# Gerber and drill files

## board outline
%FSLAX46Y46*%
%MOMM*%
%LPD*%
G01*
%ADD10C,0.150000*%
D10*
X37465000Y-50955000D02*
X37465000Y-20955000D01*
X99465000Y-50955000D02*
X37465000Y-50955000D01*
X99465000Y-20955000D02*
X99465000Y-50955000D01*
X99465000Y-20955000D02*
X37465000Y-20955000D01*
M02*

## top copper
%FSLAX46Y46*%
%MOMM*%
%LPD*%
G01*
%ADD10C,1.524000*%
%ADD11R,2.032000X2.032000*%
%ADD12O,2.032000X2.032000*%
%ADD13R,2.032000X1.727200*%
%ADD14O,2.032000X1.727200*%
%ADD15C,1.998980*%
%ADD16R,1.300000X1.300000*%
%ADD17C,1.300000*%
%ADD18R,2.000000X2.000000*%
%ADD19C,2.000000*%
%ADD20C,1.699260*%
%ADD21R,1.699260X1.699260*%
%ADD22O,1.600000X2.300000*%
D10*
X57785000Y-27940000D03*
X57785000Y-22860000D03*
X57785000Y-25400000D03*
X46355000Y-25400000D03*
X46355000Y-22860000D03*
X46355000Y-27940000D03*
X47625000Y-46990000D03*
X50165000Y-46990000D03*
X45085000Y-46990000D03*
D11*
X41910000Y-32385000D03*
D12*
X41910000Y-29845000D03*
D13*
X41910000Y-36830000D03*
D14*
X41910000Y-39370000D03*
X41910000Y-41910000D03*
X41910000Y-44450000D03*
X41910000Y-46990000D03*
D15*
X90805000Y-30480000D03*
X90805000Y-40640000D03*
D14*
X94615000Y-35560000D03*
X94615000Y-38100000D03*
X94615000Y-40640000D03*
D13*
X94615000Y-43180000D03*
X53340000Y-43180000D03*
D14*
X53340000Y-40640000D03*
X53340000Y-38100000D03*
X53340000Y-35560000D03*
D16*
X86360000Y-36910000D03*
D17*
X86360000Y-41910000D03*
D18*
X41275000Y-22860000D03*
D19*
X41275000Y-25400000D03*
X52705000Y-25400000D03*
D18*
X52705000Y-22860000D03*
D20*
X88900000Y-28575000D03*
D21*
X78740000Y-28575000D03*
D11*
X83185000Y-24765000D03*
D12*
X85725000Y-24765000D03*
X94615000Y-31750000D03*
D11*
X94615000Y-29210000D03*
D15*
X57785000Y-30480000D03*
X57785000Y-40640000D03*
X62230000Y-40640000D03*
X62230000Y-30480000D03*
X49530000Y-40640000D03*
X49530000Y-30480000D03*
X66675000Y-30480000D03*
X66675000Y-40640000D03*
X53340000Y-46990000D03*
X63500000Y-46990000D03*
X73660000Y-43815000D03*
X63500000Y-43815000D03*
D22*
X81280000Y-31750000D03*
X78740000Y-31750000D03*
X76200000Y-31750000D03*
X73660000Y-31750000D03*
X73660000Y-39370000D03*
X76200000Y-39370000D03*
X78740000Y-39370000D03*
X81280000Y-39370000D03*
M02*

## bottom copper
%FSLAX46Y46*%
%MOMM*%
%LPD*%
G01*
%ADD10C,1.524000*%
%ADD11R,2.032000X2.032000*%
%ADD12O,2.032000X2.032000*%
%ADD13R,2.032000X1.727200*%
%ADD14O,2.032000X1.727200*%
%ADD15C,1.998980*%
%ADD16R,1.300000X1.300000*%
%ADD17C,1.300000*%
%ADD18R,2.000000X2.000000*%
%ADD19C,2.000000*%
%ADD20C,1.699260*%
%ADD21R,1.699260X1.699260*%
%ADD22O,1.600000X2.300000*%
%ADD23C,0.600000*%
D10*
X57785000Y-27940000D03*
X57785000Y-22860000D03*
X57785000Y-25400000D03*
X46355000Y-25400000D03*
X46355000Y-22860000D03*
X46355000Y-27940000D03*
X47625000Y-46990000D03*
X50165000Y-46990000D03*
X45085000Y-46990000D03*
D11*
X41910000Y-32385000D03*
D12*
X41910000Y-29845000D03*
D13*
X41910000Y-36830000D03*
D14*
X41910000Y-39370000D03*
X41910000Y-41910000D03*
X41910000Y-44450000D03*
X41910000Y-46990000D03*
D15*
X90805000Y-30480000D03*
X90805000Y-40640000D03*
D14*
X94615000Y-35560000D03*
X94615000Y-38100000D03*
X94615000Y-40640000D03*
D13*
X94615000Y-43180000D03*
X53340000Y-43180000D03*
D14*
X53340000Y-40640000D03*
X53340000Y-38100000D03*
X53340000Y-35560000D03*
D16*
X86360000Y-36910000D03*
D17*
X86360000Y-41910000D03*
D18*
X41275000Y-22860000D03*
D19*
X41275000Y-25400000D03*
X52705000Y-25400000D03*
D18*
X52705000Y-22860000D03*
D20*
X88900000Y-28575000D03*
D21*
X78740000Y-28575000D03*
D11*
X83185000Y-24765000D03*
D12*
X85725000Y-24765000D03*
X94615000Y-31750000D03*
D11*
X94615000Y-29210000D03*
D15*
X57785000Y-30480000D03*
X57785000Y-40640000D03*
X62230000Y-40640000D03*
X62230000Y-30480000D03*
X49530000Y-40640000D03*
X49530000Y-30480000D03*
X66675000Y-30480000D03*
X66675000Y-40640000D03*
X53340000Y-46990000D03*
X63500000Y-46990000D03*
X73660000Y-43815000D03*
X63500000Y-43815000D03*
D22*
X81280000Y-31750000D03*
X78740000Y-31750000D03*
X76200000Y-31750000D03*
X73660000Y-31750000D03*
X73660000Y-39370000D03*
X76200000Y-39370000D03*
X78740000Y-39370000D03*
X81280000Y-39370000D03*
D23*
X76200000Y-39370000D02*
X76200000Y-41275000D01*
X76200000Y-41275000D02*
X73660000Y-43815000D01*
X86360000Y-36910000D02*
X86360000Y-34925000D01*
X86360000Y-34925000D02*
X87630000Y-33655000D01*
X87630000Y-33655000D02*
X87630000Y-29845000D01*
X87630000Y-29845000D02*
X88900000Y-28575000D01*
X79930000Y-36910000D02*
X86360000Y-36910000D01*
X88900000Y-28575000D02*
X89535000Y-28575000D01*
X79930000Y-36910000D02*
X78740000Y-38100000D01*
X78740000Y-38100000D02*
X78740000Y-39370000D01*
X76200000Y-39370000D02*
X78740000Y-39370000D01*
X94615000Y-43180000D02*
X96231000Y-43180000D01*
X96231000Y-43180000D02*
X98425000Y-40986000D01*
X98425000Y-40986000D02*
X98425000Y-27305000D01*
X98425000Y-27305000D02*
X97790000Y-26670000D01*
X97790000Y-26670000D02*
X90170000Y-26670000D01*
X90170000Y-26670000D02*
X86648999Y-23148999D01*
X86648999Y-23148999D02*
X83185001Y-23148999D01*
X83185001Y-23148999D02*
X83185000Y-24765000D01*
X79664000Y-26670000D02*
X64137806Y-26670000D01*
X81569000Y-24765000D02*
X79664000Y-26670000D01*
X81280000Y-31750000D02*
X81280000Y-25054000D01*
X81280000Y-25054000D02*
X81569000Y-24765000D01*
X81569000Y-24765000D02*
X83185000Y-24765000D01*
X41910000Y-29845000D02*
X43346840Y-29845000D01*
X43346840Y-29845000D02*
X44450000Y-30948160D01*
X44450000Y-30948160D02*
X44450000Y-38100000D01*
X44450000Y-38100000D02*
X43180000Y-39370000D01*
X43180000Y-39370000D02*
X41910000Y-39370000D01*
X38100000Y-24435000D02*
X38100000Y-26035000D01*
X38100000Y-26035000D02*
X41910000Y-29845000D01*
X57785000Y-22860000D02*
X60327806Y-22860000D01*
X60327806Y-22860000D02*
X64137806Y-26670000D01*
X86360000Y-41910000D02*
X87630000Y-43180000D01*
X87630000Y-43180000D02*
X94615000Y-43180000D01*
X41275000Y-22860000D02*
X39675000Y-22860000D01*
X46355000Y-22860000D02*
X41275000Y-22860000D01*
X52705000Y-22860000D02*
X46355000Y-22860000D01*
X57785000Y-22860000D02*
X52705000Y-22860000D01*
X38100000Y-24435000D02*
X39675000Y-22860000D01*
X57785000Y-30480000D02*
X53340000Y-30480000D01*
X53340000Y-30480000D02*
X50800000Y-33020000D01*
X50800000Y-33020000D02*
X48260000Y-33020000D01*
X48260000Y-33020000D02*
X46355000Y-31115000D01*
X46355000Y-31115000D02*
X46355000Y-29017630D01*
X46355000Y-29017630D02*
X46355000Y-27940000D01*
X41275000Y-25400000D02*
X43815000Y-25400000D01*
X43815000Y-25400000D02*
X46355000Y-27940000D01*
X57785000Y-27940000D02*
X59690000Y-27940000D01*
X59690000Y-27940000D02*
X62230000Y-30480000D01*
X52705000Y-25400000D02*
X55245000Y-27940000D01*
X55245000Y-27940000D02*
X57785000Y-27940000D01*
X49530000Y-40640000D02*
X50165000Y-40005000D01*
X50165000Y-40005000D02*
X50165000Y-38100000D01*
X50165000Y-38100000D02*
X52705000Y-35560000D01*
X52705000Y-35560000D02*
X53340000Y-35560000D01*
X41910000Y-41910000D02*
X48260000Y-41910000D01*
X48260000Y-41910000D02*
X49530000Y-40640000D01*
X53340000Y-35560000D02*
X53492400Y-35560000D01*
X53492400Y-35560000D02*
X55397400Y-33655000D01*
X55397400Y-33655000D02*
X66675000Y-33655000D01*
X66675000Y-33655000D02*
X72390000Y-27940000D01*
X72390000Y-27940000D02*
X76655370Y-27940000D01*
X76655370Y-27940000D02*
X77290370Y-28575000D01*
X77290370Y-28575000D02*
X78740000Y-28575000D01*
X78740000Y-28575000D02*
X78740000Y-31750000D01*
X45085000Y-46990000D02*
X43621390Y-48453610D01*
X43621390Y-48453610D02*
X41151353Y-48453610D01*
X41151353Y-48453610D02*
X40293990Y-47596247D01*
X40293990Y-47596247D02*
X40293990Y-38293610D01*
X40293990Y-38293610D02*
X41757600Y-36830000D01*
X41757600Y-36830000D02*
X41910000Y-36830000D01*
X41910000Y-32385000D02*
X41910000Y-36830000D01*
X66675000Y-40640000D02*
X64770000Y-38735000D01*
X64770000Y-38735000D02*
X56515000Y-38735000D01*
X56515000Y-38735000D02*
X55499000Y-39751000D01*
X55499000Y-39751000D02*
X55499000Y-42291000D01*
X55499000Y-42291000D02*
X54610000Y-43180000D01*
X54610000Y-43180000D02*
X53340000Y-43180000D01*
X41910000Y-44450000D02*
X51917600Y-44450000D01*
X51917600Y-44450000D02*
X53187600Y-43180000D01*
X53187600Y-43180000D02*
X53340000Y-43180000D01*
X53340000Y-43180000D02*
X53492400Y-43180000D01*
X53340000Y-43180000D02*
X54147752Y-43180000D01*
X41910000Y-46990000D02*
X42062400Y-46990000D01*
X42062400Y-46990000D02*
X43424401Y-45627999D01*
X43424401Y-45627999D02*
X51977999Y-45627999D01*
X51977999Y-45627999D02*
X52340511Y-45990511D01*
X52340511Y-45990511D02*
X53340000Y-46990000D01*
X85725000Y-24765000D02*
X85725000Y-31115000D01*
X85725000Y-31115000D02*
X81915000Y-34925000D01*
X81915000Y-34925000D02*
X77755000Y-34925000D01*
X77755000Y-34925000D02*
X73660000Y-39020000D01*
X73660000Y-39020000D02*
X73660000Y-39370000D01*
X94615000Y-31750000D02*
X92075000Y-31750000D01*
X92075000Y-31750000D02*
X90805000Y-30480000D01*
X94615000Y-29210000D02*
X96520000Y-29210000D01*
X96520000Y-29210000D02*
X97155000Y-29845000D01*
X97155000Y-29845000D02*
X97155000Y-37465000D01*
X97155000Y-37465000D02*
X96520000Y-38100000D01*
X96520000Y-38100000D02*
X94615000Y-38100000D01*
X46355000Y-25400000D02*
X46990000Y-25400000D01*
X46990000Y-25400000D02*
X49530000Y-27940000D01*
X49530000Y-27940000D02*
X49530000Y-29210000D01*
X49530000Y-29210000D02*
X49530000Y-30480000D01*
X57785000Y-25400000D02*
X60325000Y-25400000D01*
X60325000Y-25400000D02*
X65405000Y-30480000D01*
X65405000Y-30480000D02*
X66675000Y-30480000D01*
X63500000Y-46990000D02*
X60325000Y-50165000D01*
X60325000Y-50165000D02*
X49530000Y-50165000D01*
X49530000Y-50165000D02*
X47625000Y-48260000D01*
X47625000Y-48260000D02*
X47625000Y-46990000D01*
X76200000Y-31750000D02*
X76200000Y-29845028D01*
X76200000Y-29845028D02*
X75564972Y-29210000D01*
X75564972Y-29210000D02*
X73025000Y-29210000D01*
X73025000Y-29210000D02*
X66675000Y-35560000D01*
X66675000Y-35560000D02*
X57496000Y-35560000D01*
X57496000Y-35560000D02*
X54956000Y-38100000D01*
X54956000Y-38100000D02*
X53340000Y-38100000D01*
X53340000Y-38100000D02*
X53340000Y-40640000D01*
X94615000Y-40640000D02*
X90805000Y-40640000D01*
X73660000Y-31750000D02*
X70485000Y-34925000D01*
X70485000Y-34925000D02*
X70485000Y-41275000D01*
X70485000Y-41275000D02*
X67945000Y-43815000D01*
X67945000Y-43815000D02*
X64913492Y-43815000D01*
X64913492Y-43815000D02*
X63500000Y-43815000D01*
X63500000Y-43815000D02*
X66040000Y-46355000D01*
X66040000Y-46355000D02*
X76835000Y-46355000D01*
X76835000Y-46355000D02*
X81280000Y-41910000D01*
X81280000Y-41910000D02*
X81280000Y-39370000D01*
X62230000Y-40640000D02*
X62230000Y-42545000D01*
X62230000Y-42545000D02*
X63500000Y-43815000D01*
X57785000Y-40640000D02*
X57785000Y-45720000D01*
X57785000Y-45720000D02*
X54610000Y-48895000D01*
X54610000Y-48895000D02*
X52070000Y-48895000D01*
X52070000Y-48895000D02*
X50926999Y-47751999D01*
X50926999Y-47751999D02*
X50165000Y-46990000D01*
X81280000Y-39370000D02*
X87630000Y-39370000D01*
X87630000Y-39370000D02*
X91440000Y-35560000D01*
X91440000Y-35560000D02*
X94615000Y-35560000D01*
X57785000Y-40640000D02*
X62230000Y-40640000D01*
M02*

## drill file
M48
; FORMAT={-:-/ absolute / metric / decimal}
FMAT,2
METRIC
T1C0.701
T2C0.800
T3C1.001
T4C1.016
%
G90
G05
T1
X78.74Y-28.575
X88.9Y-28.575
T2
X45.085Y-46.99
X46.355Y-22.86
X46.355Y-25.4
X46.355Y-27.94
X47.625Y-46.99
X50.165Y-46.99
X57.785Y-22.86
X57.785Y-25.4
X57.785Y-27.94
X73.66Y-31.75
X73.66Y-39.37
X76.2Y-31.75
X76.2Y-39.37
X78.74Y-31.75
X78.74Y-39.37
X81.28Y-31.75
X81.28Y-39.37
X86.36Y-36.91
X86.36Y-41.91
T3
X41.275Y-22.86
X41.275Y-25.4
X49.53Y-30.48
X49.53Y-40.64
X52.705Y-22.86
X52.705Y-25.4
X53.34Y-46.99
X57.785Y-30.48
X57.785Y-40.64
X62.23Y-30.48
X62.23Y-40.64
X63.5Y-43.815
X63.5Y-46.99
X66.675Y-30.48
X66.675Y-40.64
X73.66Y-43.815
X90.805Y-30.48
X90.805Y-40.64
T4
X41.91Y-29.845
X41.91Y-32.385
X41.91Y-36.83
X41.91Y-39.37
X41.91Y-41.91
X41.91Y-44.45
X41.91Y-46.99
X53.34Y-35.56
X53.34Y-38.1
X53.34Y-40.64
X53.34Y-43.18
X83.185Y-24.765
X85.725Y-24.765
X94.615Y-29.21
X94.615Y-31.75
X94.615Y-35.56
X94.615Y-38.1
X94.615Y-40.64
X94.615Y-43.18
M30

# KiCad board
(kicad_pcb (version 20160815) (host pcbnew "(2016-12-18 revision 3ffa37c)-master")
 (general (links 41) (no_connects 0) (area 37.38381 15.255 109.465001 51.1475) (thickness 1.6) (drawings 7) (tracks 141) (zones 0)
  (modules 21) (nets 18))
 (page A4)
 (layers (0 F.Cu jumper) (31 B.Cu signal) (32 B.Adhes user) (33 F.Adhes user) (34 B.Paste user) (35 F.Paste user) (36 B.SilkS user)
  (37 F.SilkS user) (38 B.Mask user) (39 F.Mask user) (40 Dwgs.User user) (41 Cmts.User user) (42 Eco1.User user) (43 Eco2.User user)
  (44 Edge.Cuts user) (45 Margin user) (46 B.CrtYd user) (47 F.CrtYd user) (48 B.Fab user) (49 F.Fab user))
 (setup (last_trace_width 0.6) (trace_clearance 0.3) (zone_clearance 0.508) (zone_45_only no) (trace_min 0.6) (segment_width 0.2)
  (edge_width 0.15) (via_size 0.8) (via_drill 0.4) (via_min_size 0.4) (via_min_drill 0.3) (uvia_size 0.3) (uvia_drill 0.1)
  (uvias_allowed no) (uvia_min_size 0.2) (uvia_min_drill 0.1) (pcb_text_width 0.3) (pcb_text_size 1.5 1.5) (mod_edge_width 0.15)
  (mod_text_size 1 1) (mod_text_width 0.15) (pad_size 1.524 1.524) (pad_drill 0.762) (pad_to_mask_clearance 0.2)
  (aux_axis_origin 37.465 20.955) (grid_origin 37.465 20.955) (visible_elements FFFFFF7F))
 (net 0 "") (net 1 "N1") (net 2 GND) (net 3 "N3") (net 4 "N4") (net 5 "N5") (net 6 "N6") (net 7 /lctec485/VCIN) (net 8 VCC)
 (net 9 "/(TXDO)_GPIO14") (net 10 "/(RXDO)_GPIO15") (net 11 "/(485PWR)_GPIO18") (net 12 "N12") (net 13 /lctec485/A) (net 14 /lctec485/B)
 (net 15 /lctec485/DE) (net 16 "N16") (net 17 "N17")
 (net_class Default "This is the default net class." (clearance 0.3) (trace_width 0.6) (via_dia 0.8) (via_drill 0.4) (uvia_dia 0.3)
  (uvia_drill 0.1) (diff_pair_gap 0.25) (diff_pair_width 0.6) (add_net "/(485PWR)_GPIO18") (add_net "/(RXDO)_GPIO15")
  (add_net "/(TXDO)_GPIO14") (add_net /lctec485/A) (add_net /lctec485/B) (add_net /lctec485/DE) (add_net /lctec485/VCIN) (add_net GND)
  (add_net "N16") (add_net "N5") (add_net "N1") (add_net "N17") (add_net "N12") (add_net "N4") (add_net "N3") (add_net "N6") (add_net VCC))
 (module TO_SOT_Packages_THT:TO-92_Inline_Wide (layer F.Cu) (at 57.785 22.86 270)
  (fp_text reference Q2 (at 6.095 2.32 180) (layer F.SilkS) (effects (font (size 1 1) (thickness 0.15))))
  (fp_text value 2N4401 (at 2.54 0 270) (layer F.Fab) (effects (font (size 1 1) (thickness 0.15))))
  (pad 1 thru_hole circle (at 5.08 0) (size 1.524 1.524) (drill 0.8) (layers *.Cu *.Mask) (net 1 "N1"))
  (pad 3 thru_hole circle (at 0 0) (size 1.524 1.524) (drill 0.8) (layers *.Cu *.Mask) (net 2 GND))
  (pad 2 thru_hole circle (at 2.54 0) (size 1.524 1.524) (drill 0.8) (layers *.Cu *.Mask) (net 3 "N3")))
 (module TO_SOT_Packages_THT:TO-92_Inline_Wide (layer F.Cu) (at 46.355 22.86 270)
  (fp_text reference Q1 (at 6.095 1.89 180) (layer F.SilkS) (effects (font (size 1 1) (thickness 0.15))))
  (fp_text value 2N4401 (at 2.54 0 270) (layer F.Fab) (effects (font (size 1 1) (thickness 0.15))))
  (pad 2 thru_hole circle (at 2.54 0) (size 1.524 1.524) (drill 0.8) (layers *.Cu *.Mask) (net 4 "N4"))
  (pad 3 thru_hole circle (at 0 0) (size 1.524 1.524) (drill 0.8) (layers *.Cu *.Mask) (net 2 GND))
  (pad 1 thru_hole circle (at 5.08 0) (size 1.524 1.524) (drill 0.8) (layers *.Cu *.Mask) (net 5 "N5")))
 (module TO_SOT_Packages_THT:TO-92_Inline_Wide (layer F.Cu) (at 50.165 46.99 180)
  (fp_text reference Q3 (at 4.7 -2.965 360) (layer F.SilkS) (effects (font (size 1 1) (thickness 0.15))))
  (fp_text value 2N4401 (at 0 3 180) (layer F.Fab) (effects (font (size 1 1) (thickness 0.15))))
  (pad 2 thru_hole circle (at 2.54 0 270) (size 1.524 1.524) (drill 0.8) (layers *.Cu *.Mask) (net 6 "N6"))
  (pad 3 thru_hole circle (at 0 0 270) (size 1.524 1.524) (drill 0.8) (layers *.Cu *.Mask) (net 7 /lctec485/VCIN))
  (pad 1 thru_hole circle (at 5.08 0 270) (size 1.524 1.524) (drill 0.8) (layers *.Cu *.Mask) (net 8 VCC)))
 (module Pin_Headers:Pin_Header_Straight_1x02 (layer F.Cu) (at 41.91 32.385 180)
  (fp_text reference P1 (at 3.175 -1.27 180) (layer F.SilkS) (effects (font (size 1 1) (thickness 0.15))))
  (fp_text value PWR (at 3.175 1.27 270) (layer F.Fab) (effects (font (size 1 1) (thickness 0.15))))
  (pad 1 thru_hole rect (at 0 0 180) (size 2.032 2.032) (drill 1.016) (layers *.Cu *.Mask) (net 8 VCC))
  (pad 2 thru_hole oval (at 0 2.54 180) (size 2.032 2.032) (drill 1.016) (layers *.Cu *.Mask) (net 2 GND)))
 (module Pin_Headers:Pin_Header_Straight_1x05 (layer F.Cu) (at 41.91 36.83)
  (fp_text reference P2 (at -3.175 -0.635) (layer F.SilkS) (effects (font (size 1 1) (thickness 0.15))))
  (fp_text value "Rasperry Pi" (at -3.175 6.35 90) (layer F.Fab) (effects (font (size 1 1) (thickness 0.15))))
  (pad 1 thru_hole rect (at 0 0) (size 2.032 1.7272) (drill 1.016) (layers *.Cu *.Mask) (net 8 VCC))
  (pad 2 thru_hole oval (at 0 2.54) (size 2.032 1.7272) (drill 1.016) (layers *.Cu *.Mask) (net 2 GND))
  (pad 3 thru_hole oval (at 0 5.08) (size 2.032 1.7272) (drill 1.016) (layers *.Cu *.Mask) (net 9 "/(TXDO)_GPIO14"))
  (pad 4 thru_hole oval (at 0 7.62) (size 2.032 1.7272) (drill 1.016) (layers *.Cu *.Mask) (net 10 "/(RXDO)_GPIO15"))
  (pad 5 thru_hole oval (at 0 10.16) (size 2.032 1.7272) (drill 1.016) (layers *.Cu *.Mask) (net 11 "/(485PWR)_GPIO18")))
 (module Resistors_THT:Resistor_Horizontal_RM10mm (layer F.Cu) (at 90.805 30.48 270)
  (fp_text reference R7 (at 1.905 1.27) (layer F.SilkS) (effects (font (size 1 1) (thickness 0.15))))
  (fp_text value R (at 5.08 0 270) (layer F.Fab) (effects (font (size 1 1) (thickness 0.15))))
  (pad 1 thru_hole circle (at 0 0 270) (size 1.99898 1.99898) (drill 1.00076) (layers *.Cu *.SilkS *.Mask) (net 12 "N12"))
  (pad 2 thru_hole circle (at 10.16 0 270) (size 1.99898 1.99898) (drill 1.00076) (layers *.Cu *.SilkS *.Mask) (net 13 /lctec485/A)))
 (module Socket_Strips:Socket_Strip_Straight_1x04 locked (layer F.Cu) (at 94.615 43.18 90)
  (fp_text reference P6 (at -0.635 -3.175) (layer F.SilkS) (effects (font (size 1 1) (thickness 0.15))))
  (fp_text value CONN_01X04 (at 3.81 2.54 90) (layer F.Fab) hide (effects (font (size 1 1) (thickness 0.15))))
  (pad 4 thru_hole oval (at 7.62 0 90) (size 1.7272 2.032) (drill 1.016) (layers *.Cu *.Mask) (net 7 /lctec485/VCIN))
  (pad 3 thru_hole oval (at 5.08 0 90) (size 1.7272 2.032) (drill 1.016) (layers *.Cu *.Mask) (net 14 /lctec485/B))
  (pad 2 thru_hole oval (at 2.54 0 90) (size 1.7272 2.032) (drill 1.016) (layers *.Cu *.Mask) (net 13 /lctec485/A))
  (pad 1 thru_hole rect (at 0 0 90) (size 1.7272 2.032) (drill 1.016) (layers *.Cu *.Mask) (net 2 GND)))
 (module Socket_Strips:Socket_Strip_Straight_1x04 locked (layer F.Cu) (at 53.34 43.18 90)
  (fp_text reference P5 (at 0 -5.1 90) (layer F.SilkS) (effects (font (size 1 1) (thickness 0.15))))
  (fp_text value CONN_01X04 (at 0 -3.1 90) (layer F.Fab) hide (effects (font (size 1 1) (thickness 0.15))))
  (pad 1 thru_hole rect (at 0 0 90) (size 1.7272 2.032) (drill 1.016) (layers *.Cu *.Mask) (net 10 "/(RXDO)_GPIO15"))
  (pad 2 thru_hole oval (at 2.54 0 90) (size 1.7272 2.032) (drill 1.016) (layers *.Cu *.Mask) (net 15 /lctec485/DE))
  (pad 3 thru_hole oval (at 5.08 0 90) (size 1.7272 2.032) (drill 1.016) (layers *.Cu *.Mask) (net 15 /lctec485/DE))
  (pad 4 thru_hole oval (at 7.62 0 90) (size 1.7272 2.032) (drill 1.016) (layers *.Cu *.Mask) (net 9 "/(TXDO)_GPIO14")))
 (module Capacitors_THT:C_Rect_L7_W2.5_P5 (layer F.Cu) (at 86.36 36.91 270)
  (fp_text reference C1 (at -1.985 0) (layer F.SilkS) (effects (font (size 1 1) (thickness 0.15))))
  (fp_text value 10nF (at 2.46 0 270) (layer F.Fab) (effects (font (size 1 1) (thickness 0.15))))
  (pad 1 thru_hole rect (at 0 0 270) (size 1.3 1.3) (drill 0.8) (layers *.Cu *.Mask) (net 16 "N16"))
  (pad 2 thru_hole circle (at 5 0 270) (size 1.3 1.3) (drill 0.8) (layers *.Cu *.Mask) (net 2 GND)))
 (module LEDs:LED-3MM (layer F.Cu) (at 41.275 22.86 270)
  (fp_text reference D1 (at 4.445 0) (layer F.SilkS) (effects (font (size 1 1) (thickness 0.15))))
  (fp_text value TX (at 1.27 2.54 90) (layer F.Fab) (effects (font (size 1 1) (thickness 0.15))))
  (pad 1 thru_hole rect (at 0 0) (size 2 2) (drill 1.00076) (layers *.Cu *.Mask) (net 2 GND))
  (pad 2 thru_hole circle (at 2.54 0 270) (size 2 2) (drill 1.00076) (layers *.Cu *.Mask) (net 5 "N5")))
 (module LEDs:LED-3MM (layer F.Cu) (at 52.705 22.86 270)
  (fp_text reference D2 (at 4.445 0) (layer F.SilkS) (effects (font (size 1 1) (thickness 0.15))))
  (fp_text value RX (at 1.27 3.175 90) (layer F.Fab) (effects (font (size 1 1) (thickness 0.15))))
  (pad 2 thru_hole circle (at 2.54 0 270) (size 2 2) (drill 1.00076) (layers *.Cu *.Mask) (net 1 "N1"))
  (pad 1 thru_hole rect (at 0 0) (size 2 2) (drill 1.00076) (layers *.Cu *.Mask) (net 2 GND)))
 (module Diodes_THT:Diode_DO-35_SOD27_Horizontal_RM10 (layer F.Cu) (at 78.73948 28.57754)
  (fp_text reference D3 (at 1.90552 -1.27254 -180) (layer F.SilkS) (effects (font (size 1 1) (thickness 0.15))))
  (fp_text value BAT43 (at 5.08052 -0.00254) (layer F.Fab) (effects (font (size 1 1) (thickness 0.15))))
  (pad 2 thru_hole circle (at 10.16052 -0.00254 180) (size 1.69926 1.69926) (drill 0.70104) (layers *.Cu *.Mask) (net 16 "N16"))
  (pad 1 thru_hole rect (at 0.00052 -0.00254 180) (size 1.69926 1.69926) (drill 0.70104) (layers *.Cu *.Mask) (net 9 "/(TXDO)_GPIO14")))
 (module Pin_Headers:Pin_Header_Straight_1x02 (layer F.Cu) (at 83.185 24.765 90)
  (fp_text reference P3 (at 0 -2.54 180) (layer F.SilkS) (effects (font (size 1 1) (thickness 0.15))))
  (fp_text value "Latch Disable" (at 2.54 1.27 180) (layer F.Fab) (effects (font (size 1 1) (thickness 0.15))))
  (pad 1 thru_hole rect (at 0 0 90) (size 2.032 2.032) (drill 1.016) (layers *.Cu *.Mask) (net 2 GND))
  (pad 2 thru_hole oval (at 0 2.54 90) (size 2.032 2.032) (drill 1.016) (layers *.Cu *.Mask) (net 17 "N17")))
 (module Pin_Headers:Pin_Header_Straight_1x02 (layer F.Cu) (at 94.615 29.21)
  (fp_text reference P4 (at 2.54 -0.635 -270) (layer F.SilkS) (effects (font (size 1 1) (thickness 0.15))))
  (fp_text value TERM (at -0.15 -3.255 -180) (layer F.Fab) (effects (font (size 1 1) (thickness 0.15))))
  (pad 2 thru_hole oval (at 0 2.54) (size 2.032 2.032) (drill 1.016) (layers *.Cu *.Mask) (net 12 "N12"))
  (pad 1 thru_hole rect (at 0 0) (size 2.032 2.032) (drill 1.016) (layers *.Cu *.Mask) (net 14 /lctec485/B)))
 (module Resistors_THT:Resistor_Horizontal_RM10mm (layer F.Cu) (at 57.785 30.48 270)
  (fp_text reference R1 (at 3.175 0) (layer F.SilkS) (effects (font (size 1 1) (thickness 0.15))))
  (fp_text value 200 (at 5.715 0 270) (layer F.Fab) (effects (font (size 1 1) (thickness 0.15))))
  (pad 1 thru_hole circle (at 0 0 270) (size 1.99898 1.99898) (drill 1.00076) (layers *.Cu *.SilkS *.Mask) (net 5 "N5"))
  (pad 2 thru_hole circle (at 10.16 0 270) (size 1.99898 1.99898) (drill 1.00076) (layers *.Cu *.SilkS *.Mask) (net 7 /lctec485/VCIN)))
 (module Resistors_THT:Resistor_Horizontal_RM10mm (layer F.Cu) (at 62.23 30.48 270)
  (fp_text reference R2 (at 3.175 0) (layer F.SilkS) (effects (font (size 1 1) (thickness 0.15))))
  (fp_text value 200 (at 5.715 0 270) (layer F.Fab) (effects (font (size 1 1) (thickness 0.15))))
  (pad 2 thru_hole circle (at 10.16 0 270) (size 1.99898 1.99898) (drill 1.00076) (layers *.Cu *.SilkS *.Mask) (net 7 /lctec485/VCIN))
  (pad 1 thru_hole circle (at 0 0 270) (size 1.99898 1.99898) (drill 1.00076) (layers *.Cu *.SilkS *.Mask) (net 1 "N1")))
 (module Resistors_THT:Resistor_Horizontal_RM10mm (layer F.Cu) (at 49.53 30.48 270)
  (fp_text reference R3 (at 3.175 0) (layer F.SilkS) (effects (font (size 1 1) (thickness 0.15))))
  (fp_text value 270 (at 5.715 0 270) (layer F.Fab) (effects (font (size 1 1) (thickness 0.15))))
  (pad 2 thru_hole circle (at 10.16 0 270) (size 1.99898 1.99898) (drill 1.00076) (layers *.Cu *.SilkS *.Mask) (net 9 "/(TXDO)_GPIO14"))
  (pad 1 thru_hole circle (at 0 0 270) (size 1.99898 1.99898) (drill 1.00076) (layers *.Cu *.SilkS *.Mask) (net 4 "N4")))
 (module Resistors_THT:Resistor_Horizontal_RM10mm (layer F.Cu) (at 66.675 30.48 270)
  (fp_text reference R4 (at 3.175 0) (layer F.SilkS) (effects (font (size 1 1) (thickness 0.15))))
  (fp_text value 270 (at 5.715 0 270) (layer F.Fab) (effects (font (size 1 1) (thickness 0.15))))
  (pad 1 thru_hole circle (at 0 0 270) (size 1.99898 1.99898) (drill 1.00076) (layers *.Cu *.SilkS *.Mask) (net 3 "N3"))
  (pad 2 thru_hole circle (at 10.16 0 270) (size 1.99898 1.99898) (drill 1.00076) (layers *.Cu *.SilkS *.Mask) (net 10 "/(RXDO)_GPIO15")))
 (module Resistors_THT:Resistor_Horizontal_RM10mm (layer F.Cu) (at 63.5 46.99 180)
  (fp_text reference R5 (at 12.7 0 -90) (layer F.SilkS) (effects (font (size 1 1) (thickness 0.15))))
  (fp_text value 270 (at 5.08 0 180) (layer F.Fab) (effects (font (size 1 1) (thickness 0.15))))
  (pad 2 thru_hole circle (at 10.16 0 180) (size 1.99898 1.99898) (drill 1.00076) (layers *.Cu *.SilkS *.Mask) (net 11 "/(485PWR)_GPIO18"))
  (pad 1 thru_hole circle (at 0 0 180) (size 1.99898 1.99898) (drill 1.00076) (layers *.Cu *.SilkS *.Mask) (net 6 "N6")))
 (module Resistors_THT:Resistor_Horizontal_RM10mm (layer F.Cu) (at 73.66 43.815 180)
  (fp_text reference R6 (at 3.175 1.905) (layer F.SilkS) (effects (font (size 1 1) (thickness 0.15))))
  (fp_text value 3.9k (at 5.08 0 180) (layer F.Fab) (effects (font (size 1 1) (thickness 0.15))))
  (pad 1 thru_hole circle (at 0 0 180) (size 1.99898 1.99898) (drill 1.00076) (layers *.Cu *.SilkS *.Mask) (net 16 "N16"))
  (pad 2 thru_hole circle (at 10.16 0 180) (size 1.99898 1.99898) (drill 1.00076) (layers *.Cu *.SilkS *.Mask) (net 7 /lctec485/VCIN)))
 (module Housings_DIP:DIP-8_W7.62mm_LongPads (layer F.Cu) (at 81.28 31.75 270)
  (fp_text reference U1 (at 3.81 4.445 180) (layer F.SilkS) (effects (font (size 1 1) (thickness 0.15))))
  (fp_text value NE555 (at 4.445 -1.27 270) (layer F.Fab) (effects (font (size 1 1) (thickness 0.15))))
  (pad 1 thru_hole oval (at 0 0 270) (size 2.3 1.6) (drill 0.8) (layers *.Cu *.Mask) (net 2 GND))
  (pad 2 thru_hole oval (at 0 2.54 270) (size 2.3 1.6) (drill 0.8) (layers *.Cu *.Mask) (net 9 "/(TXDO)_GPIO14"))
  (pad 3 thru_hole oval (at 0 5.08 270) (size 2.3 1.6) (drill 0.8) (layers *.Cu *.Mask) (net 15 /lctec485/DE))
  (pad 4 thru_hole oval (at 0 7.62 270) (size 2.3 1.6) (drill 0.8) (layers *.Cu *.Mask) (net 7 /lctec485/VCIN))
  (pad 5 thru_hole oval (at 7.62 7.62 270) (size 2.3 1.6) (drill 0.8) (layers *.Cu *.Mask) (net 17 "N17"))
  (pad 6 thru_hole oval (at 7.62 5.08 270) (size 2.3 1.6) (drill 0.8) (layers *.Cu *.Mask) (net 16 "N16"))
  (pad 7 thru_hole oval (at 7.62 2.54 270) (size 2.3 1.6) (drill 0.8) (layers *.Cu *.Mask) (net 16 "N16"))
  (pad 8 thru_hole oval (at 7.62 0 270) (size 2.3 1.6) (drill 0.8) (layers *.Cu *.Mask) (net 7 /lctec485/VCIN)))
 (gr_line (start 37.465 50.955) (end 37.465 20.955) (layer Edge.Cuts) (width 0.15))
 (gr_line (start 99.465 50.955) (end 37.465 50.955) (layer Edge.Cuts) (width 0.15))
 (gr_line (start 99.465 20.955) (end 99.465 50.955) (layer Edge.Cuts) (width 0.15))
 (gr_line (start 99.465 20.955) (end 37.465 20.955) (layer Edge.Cuts) (width 0.15))
 (segment (start 76.2 39.37) (end 76.2 41.275) (width 0.6) (layer B.Cu) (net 16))
 (segment (start 76.2 41.275) (end 73.66 43.815) (width 0.6) (layer B.Cu) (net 16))
 (segment (start 86.36 36.91) (end 86.36 34.925) (width 0.6) (layer B.Cu) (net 16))
 (segment (start 86.36 34.925) (end 87.63 33.655) (width 0.6) (layer B.Cu) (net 16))
 (segment (start 87.63 33.655) (end 87.63 29.845) (width 0.6) (layer B.Cu) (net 16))
 (segment (start 87.63 29.845) (end 88.9 28.575) (width 0.6) (layer B.Cu) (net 16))
 (segment (start 79.93 36.91) (end 86.36 36.91) (width 0.6) (layer B.Cu) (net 16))
 (segment (start 88.9 28.575) (end 89.535 28.575) (width 0.6) (layer B.Cu) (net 16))
 (segment (start 79.93 36.91) (end 78.74 38.1) (width 0.6) (layer B.Cu) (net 16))
 (segment (start 78.74 38.1) (end 78.74 39.37) (width 0.6) (layer B.Cu) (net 16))
 (segment (start 76.2 39.37) (end 78.74 39.37) (width 0.6) (layer B.Cu) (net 16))
 (segment (start 94.615 43.18) (end 96.231 43.18) (width 0.6) (layer B.Cu) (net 2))
 (segment (start 96.231 43.18) (end 98.425 40.986) (width 0.6) (layer B.Cu) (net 2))
 (segment (start 98.425 40.986) (end 98.425 27.305) (width 0.6) (layer B.Cu) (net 2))
 (segment (start 98.425 27.305) (end 97.79 26.67) (width 0.6) (layer B.Cu) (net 2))
 (segment (start 97.79 26.67) (end 90.17 26.67) (width 0.6) (layer B.Cu) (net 2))
 (segment (start 90.17 26.67) (end 86.648999 23.148999) (width 0.6) (layer B.Cu) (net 2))
 (segment (start 86.648999 23.148999) (end 83.185001 23.148999) (width 0.6) (layer B.Cu) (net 2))
 (segment (start 83.185001 23.148999) (end 83.185 24.765) (width 0.6) (layer B.Cu) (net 2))
 (segment (start 79.664 26.67) (end 64.137806 26.67) (width 0.6) (layer B.Cu) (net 2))
 (segment (start 81.569 24.765) (end 79.664 26.67) (width 0.6) (layer B.Cu) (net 2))
 (segment (start 81.28 31.75) (end 81.28 25.054) (width 0.6) (layer B.Cu) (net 2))
 (segment (start 81.28 25.054) (end 81.569 24.765) (width 0.6) (layer B.Cu) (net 2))
 (segment (start 81.569 24.765) (end 83.185 24.765) (width 0.6) (layer B.Cu) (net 2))
 (segment (start 41.91 29.845) (end 43.34684 29.845) (width 0.6) (layer B.Cu) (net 2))
 (segment (start 43.34684 29.845) (end 44.45 30.94816) (width 0.6) (layer B.Cu) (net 2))
 (segment (start 44.45 30.94816) (end 44.45 38.1) (width 0.6) (layer B.Cu) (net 2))
 (segment (start 44.45 38.1) (end 43.18 39.37) (width 0.6) (layer B.Cu) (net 2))
 (segment (start 43.18 39.37) (end 41.91 39.37) (width 0.6) (layer B.Cu) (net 2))
 (segment (start 38.1 24.435) (end 38.1 26.035) (width 0.6) (layer B.Cu) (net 2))
 (segment (start 38.1 26.035) (end 41.91 29.845) (width 0.6) (layer B.Cu) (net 2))
 (segment (start 57.785 22.86) (end 60.327806 22.86) (width 0.6) (layer B.Cu) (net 2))
 (segment (start 60.327806 22.86) (end 64.137806 26.67) (width 0.6) (layer B.Cu) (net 2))
 (segment (start 86.36 41.91) (end 87.63 43.18) (width 0.6) (layer B.Cu) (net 2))
 (segment (start 87.63 43.18) (end 94.615 43.18) (width 0.6) (layer B.Cu) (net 2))
 (segment (start 41.275 22.86) (end 39.675 22.86) (width 0.6) (layer B.Cu) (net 2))
 (segment (start 46.355 22.86) (end 41.275 22.86) (width 0.6) (layer B.Cu) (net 2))
 (segment (start 52.705 22.86) (end 46.355 22.86) (width 0.6) (layer B.Cu) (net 2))
 (segment (start 57.785 22.86) (end 52.705 22.86) (width 0.6) (layer B.Cu) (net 2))
 (segment (start 38.1 24.435) (end 39.675 22.86) (width 0.6) (layer B.Cu) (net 2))
 (segment (start 57.785 30.48) (end 53.34 30.48) (width 0.6) (layer B.Cu) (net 5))
 (segment (start 53.34 30.48) (end 50.8 33.02) (width 0.6) (layer B.Cu) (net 5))
 (segment (start 50.8 33.02) (end 48.26 33.02) (width 0.6) (layer B.Cu) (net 5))
 (segment (start 48.26 33.02) (end 46.355 31.115) (width 0.6) (layer B.Cu) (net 5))
 (segment (start 46.355 31.115) (end 46.355 29.01763) (width 0.6) (layer B.Cu) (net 5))
 (segment (start 46.355 29.01763) (end 46.355 27.94) (width 0.6) (layer B.Cu) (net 5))
 (segment (start 41.275 25.4) (end 43.815 25.4) (width 0.6) (layer B.Cu) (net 5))
 (segment (start 43.815 25.4) (end 46.355 27.94) (width 0.6) (layer B.Cu) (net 5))
 (segment (start 57.785 27.94) (end 59.69 27.94) (width 0.6) (layer B.Cu) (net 1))
 (segment (start 59.69 27.94) (end 62.23 30.48) (width 0.6) (layer B.Cu) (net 1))
 (segment (start 52.705 25.4) (end 55.245 27.94) (width 0.6) (layer B.Cu) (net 1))
 (segment (start 55.245 27.94) (end 57.785 27.94) (width 0.6) (layer B.Cu) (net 1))
 (segment (start 49.53 40.64) (end 50.165 40.005) (width 0.6) (layer B.Cu) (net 9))
 (segment (start 50.165 40.005) (end 50.165 38.1) (width 0.6) (layer B.Cu) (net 9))
 (segment (start 50.165 38.1) (end 52.705 35.56) (width 0.6) (layer B.Cu) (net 9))
 (segment (start 52.705 35.56) (end 53.34 35.56) (width 0.6) (layer B.Cu) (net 9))
 (segment (start 41.91 41.91) (end 48.26 41.91) (width 0.6) (layer B.Cu) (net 9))
 (segment (start 48.26 41.91) (end 49.53 40.64) (width 0.6) (layer B.Cu) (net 9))
 (segment (start 53.34 35.56) (end 53.4924 35.56) (width 0.6) (layer B.Cu) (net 9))
 (segment (start 53.4924 35.56) (end 55.3974 33.655) (width 0.6) (layer B.Cu) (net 9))
 (segment (start 55.3974 33.655) (end 66.675 33.655) (width 0.6) (layer B.Cu) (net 9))
 (segment (start 66.675 33.655) (end 72.39 27.94) (width 0.6) (layer B.Cu) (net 9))
 (segment (start 72.39 27.94) (end 76.65537 27.94) (width 0.6) (layer B.Cu) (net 9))
 (segment (start 76.65537 27.94) (end 77.29037 28.575) (width 0.6) (layer B.Cu) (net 9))
 (segment (start 77.29037 28.575) (end 78.74 28.575) (width 0.6) (layer B.Cu) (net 9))
 (segment (start 78.74 28.575) (end 78.74 31.75) (width 0.6) (layer B.Cu) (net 9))
 (segment (start 45.085 46.99) (end 43.62139 48.45361) (width 0.6) (layer B.Cu) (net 8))
 (segment (start 43.62139 48.45361) (end 41.151353 48.45361) (width 0.6) (layer B.Cu) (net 8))
 (segment (start 41.151353 48.45361) (end 40.29399 47.596247) (width 0.6) (layer B.Cu) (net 8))
 (segment (start 40.29399 47.596247) (end 40.29399 38.29361) (width 0.6) (layer B.Cu) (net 8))
 (segment (start 40.29399 38.29361) (end 41.7576 36.83) (width 0.6) (layer B.Cu) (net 8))
 (segment (start 41.7576 36.83) (end 41.91 36.83) (width 0.6) (layer B.Cu) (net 8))
 (segment (start 41.91 32.385) (end 41.91 36.83) (width 0.6) (layer B.Cu) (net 8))
 (segment (start 66.675 40.64) (end 64.77 38.735) (width 0.6) (layer B.Cu) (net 10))
 (segment (start 64.77 38.735) (end 56.515 38.735) (width 0.6) (layer B.Cu) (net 10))
 (segment (start 56.515 38.735) (end 55.499 39.751) (width 0.6) (layer B.Cu) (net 10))
 (segment (start 55.499 39.751) (end 55.499 42.291) (width 0.6) (layer B.Cu) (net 10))
 (segment (start 55.499 42.291) (end 54.61 43.18) (width 0.6) (layer B.Cu) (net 10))
 (segment (start 54.61 43.18) (end 53.34 43.18) (width 0.6) (layer B.Cu) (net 10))
 (segment (start 41.91 44.45) (end 51.9176 44.45) (width 0.6) (layer B.Cu) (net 10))
 (segment (start 51.9176 44.45) (end 53.1876 43.18) (width 0.6) (layer B.Cu) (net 10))
 (segment (start 53.1876 43.18) (end 53.34 43.18) (width 0.6) (layer B.Cu) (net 10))
 (segment (start 53.34 43.18) (end 53.4924 43.18) (width 0.6) (layer B.Cu) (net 10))
 (segment (start 53.34 43.18) (end 54.147752 43.18) (width 0.6) (layer B.Cu) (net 10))
 (segment (start 41.91 46.99) (end 42.0624 46.99) (width 0.6) (layer B.Cu) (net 11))
 (segment (start 42.0624 46.99) (end 43.424401 45.627999) (width 0.6) (layer B.Cu) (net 11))
 (segment (start 43.424401 45.627999) (end 51.977999 45.627999) (width 0.6) (layer B.Cu) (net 11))
 (segment (start 51.977999 45.627999) (end 52.340511 45.990511) (width 0.6) (layer B.Cu) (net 11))
 (segment (start 52.340511 45.990511) (end 53.34 46.99) (width 0.6) (layer B.Cu) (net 11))
 (segment (start 85.725 24.765) (end 85.725 31.115) (width 0.6) (layer B.Cu) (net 17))
 (segment (start 85.725 31.115) (end 81.915 34.925) (width 0.6) (layer B.Cu) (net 17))
 (segment (start 81.915 34.925) (end 77.755 34.925) (width 0.6) (layer B.Cu) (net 17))
 (segment (start 77.755 34.925) (end 73.66 39.02) (width 0.6) (layer B.Cu) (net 17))
 (segment (start 73.66 39.02) (end 73.66 39.37) (width 0.6) (layer B.Cu) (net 17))
 (segment (start 94.615 31.75) (end 92.075 31.75) (width 0.6) (layer B.Cu) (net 12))
 (segment (start 92.075 31.75) (end 90.805 30.48) (width 0.6) (layer B.Cu) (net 12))
 (segment (start 94.615 29.21) (end 96.52 29.21) (width 0.6) (layer B.Cu) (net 14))
 (segment (start 96.52 29.21) (end 97.155 29.845) (width 0.6) (layer B.Cu) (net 14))
 (segment (start 97.155 29.845) (end 97.155 37.465) (width 0.6) (layer B.Cu) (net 14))
 (segment (start 97.155 37.465) (end 96.52 38.1) (width 0.6) (layer B.Cu) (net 14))
 (segment (start 96.52 38.1) (end 94.615 38.1) (width 0.6) (layer B.Cu) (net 14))
 (segment (start 46.355 25.4) (end 46.99 25.4) (width 0.6) (layer B.Cu) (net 4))
 (segment (start 46.99 25.4) (end 49.53 27.94) (width 0.6) (layer B.Cu) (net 4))
 (segment (start 49.53 27.94) (end 49.53 29.21) (width 0.6) (layer B.Cu) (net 4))
 (segment (start 49.53 29.21) (end 49.53 30.48) (width 0.6) (layer B.Cu) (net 4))
 (segment (start 57.785 25.4) (end 60.325 25.4) (width 0.6) (layer B.Cu) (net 3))
 (segment (start 60.325 25.4) (end 65.405 30.48) (width 0.6) (layer B.Cu) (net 3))
 (segment (start 65.405 30.48) (end 66.675 30.48) (width 0.6) (layer B.Cu) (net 3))
 (segment (start 63.5 46.99) (end 60.325 50.165) (width 0.6) (layer B.Cu) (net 6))
 (segment (start 60.325 50.165) (end 49.53 50.165) (width 0.6) (layer B.Cu) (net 6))
 (segment (start 49.53 50.165) (end 47.625 48.26) (width 0.6) (layer B.Cu) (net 6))
 (segment (start 47.625 48.26) (end 47.625 46.99) (width 0.6) (layer B.Cu) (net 6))
 (segment (start 76.2 31.75) (end 76.2 29.845028) (width 0.6) (layer B.Cu) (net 15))
 (segment (start 76.2 29.845028) (end 75.564972 29.21) (width 0.6) (layer B.Cu) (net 15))
 (segment (start 75.564972 29.21) (end 73.025 29.21) (width 0.6) (layer B.Cu) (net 15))
 (segment (start 73.025 29.21) (end 66.675 35.56) (width 0.6) (layer B.Cu) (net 15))
 (segment (start 66.675 35.56) (end 57.496 35.56) (width 0.6) (layer B.Cu) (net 15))
 (segment (start 57.496 35.56) (end 54.956 38.1) (width 0.6) (layer B.Cu) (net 15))
 (segment (start 54.956 38.1) (end 53.34 38.1) (width 0.6) (layer B.Cu) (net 15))
 (segment (start 53.34 38.1) (end 53.34 40.64) (width 0.6) (layer B.Cu) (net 15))
 (segment (start 94.615 40.64) (end 90.805 40.64) (width 0.6) (layer B.Cu) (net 13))
 (segment (start 73.66 31.75) (end 70.485 34.925) (width 0.6) (layer B.Cu) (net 7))
 (segment (start 70.485 34.925) (end 70.485 41.275) (width 0.6) (layer B.Cu) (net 7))
 (segment (start 70.485 41.275) (end 67.945 43.815) (width 0.6) (layer B.Cu) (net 7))
 (segment (start 67.945 43.815) (end 64.913492 43.815) (width 0.6) (layer B.Cu) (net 7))
 (segment (start 64.913492 43.815) (end 63.5 43.815) (width 0.6) (layer B.Cu) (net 7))
 (segment (start 63.5 43.815) (end 66.04 46.355) (width 0.6) (layer B.Cu) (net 7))
 (segment (start 66.04 46.355) (end 76.835 46.355) (width 0.6) (layer B.Cu) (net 7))
 (segment (start 76.835 46.355) (end 81.28 41.91) (width 0.6) (layer B.Cu) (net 7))
 (segment (start 81.28 41.91) (end 81.28 39.37) (width 0.6) (layer B.Cu) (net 7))
 (segment (start 62.23 40.64) (end 62.23 42.545) (width 0.6) (layer B.Cu) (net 7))
 (segment (start 62.23 42.545) (end 63.5 43.815) (width 0.6) (layer B.Cu) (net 7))
 (segment (start 57.785 40.64) (end 57.785 45.72) (width 0.6) (layer B.Cu) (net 7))
 (segment (start 57.785 45.72) (end 54.61 48.895) (width 0.6) (layer B.Cu) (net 7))
 (segment (start 54.61 48.895) (end 52.07 48.895) (width 0.6) (layer B.Cu) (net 7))
 (segment (start 52.07 48.895) (end 50.926999 47.751999) (width 0.6) (layer B.Cu) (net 7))
 (segment (start 50.926999 47.751999) (end 50.165 46.99) (width 0.6) (layer B.Cu) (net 7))
 (segment (start 81.28 39.37) (end 87.63 39.37) (width 0.6) (layer B.Cu) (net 7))
 (segment (start 87.63 39.37) (end 91.44 35.56) (width 0.6) (layer B.Cu) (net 7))
 (segment (start 91.44 35.56) (end 94.615 35.56) (width 0.6) (layer B.Cu) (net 7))
 (segment (start 57.785 40.64) (end 62.23 40.64) (width 0.6) (layer B.Cu) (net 7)))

